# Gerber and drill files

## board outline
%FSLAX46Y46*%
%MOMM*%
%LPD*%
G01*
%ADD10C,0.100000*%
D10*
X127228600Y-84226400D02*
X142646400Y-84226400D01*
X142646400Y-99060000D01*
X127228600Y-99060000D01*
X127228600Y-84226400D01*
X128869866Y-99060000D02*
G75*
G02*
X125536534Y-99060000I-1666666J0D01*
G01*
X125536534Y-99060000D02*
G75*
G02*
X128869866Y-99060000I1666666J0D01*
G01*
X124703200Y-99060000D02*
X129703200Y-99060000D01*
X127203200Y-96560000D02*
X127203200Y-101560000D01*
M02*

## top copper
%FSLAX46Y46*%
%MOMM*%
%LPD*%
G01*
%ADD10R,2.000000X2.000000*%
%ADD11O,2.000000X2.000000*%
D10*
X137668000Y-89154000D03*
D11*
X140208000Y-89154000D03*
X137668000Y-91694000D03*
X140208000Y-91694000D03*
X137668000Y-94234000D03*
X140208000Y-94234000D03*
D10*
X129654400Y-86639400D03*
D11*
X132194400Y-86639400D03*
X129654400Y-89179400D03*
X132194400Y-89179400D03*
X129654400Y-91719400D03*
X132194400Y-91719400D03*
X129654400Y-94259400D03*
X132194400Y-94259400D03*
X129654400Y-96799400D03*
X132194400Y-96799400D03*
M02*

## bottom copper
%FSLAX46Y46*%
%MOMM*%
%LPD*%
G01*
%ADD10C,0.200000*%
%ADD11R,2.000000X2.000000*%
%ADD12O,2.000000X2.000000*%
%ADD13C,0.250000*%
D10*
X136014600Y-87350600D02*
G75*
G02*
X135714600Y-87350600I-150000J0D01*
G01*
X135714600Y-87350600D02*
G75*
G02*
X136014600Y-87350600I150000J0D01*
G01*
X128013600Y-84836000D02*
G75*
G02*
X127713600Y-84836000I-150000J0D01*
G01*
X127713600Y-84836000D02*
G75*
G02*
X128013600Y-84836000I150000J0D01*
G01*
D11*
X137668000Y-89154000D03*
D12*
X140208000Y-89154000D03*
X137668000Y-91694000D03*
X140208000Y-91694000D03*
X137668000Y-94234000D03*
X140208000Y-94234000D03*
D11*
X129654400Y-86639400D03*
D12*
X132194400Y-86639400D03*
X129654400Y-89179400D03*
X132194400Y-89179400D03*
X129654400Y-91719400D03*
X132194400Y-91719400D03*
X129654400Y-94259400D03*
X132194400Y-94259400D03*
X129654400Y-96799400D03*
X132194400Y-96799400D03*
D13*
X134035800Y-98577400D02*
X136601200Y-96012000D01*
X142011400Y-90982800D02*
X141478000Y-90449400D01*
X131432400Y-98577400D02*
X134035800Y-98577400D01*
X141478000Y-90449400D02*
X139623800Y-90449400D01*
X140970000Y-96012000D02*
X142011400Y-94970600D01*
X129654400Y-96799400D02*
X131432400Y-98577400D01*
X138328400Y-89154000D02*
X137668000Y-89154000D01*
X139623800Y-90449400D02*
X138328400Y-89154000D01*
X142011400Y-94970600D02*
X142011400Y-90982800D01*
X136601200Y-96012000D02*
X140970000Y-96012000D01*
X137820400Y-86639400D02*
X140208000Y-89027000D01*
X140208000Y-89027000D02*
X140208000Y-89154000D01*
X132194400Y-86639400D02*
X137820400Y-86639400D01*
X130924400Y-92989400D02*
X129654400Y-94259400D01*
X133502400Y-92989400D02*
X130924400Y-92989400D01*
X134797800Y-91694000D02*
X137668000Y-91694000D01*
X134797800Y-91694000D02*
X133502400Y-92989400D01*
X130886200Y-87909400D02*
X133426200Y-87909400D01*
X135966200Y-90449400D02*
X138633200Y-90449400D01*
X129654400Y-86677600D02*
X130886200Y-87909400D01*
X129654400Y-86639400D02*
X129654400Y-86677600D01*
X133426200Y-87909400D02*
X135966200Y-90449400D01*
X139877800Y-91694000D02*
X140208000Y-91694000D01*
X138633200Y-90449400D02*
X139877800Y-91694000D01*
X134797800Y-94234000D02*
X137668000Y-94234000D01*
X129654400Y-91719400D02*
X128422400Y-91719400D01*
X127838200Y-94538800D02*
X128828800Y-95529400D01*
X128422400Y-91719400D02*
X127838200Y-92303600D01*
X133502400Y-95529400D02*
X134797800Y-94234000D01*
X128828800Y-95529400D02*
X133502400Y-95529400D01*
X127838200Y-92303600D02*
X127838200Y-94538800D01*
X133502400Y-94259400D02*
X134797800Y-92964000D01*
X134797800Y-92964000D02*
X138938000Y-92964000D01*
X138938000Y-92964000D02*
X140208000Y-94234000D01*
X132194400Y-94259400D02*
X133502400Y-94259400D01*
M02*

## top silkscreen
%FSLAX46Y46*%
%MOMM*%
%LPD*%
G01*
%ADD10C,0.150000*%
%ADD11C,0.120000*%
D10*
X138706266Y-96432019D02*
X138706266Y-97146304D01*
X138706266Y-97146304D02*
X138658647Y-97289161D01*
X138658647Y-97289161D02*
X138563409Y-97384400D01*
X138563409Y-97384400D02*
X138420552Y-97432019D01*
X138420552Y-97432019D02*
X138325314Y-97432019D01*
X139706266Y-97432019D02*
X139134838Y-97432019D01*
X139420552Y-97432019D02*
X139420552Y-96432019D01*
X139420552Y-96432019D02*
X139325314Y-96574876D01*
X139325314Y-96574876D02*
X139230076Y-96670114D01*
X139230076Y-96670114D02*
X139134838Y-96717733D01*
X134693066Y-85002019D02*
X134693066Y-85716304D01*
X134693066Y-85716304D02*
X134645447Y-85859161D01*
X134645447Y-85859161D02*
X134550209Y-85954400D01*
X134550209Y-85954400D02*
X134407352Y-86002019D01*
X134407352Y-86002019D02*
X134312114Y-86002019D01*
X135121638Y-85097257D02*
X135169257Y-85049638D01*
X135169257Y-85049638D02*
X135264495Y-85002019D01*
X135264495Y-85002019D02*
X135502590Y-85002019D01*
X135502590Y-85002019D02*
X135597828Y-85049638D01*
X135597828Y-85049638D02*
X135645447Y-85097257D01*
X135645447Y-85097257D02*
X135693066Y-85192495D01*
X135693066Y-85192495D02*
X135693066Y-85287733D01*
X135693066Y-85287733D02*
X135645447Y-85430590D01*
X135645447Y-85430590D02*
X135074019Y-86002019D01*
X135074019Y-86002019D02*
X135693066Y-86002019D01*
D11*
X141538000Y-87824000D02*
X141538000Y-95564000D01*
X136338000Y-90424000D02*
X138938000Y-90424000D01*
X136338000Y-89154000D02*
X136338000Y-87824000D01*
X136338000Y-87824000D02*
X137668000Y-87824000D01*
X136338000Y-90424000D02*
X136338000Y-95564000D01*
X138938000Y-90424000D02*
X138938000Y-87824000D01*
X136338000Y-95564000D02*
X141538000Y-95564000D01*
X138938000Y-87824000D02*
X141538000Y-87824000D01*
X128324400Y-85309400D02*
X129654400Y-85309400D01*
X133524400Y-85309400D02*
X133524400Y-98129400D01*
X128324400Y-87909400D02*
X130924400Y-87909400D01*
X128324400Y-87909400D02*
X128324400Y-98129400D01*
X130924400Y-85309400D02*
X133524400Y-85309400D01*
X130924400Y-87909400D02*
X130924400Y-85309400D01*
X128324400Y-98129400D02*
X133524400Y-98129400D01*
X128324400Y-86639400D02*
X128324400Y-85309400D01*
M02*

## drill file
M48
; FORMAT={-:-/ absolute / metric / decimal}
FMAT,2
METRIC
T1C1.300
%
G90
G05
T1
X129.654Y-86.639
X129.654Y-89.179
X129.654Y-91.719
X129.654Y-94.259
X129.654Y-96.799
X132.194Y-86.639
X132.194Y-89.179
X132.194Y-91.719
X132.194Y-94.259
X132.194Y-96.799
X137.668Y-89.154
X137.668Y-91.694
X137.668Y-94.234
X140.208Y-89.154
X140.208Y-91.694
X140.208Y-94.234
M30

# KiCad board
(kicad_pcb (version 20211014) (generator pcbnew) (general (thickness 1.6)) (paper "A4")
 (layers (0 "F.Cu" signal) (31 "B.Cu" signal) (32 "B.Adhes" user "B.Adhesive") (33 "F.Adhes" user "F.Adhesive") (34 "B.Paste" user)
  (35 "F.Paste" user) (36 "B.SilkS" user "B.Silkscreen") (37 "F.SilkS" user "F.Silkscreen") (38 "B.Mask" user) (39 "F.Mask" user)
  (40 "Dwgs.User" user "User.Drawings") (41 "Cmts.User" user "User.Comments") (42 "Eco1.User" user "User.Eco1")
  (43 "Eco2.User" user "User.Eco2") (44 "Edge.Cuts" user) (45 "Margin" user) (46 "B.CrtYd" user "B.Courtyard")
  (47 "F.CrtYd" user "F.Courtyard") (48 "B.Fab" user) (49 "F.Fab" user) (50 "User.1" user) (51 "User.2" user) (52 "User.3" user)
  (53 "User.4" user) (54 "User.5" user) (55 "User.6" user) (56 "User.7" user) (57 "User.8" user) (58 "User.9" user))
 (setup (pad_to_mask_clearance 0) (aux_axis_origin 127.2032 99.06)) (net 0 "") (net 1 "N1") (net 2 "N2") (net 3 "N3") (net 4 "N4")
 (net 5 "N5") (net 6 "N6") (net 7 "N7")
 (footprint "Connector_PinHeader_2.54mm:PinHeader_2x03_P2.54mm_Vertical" (layer "F.Cu") (at 137.668 89.154)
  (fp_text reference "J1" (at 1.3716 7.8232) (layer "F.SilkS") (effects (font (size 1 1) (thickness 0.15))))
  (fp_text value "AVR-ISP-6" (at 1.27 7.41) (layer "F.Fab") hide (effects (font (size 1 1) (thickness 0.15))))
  (fp_line (start 3.87 -1.33) (end 3.87 6.41) (layer "F.SilkS") (width 0.12))
  (fp_line (start -1.33 1.27) (end 1.27 1.27) (layer "F.SilkS") (width 0.12))
  (fp_line (start -1.33 0) (end -1.33 -1.33) (layer "F.SilkS") (width 0.12))
  (fp_line (start -1.33 -1.33) (end 0 -1.33) (layer "F.SilkS") (width 0.12))
  (fp_line (start -1.33 1.27) (end -1.33 6.41) (layer "F.SilkS") (width 0.12))
  (fp_line (start 1.27 1.27) (end 1.27 -1.33) (layer "F.SilkS") (width 0.12))
  (fp_line (start -1.33 6.41) (end 3.87 6.41) (layer "F.SilkS") (width 0.12))
  (fp_line (start 1.27 -1.33) (end 3.87 -1.33) (layer "F.SilkS") (width 0.12))
  (pad "1" thru_hole rect locked (at 0 0) (size 2 2) (drill 1.3) (layers *.Cu *.Mask) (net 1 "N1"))
  (pad "2" thru_hole oval locked (at 2.54 0) (size 2 2) (drill 1.3) (layers *.Cu *.Mask) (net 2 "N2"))
  (pad "3" thru_hole oval locked (at 0 2.54) (size 2 2) (drill 1.3) (layers *.Cu *.Mask) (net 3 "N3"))
  (pad "4" thru_hole oval locked (at 2.54 2.54) (size 2 2) (drill 1.3) (layers *.Cu *.Mask) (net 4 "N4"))
  (pad "5" thru_hole oval locked (at 0 5.08) (size 2 2) (drill 1.3) (layers *.Cu *.Mask) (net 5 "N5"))
  (pad "6" thru_hole oval locked (at 2.54 5.08) (size 2 2) (drill 1.3) (layers *.Cu *.Mask) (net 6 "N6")))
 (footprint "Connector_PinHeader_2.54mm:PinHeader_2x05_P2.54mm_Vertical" (layer "F.Cu") (at 129.6544 86.6394)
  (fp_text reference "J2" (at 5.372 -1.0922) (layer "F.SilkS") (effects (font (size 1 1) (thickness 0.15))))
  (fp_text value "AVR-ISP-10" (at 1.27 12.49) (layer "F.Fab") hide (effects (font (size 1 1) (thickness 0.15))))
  (fp_line (start -1.33 -1.33) (end 0 -1.33) (layer "F.SilkS") (width 0.12))
  (fp_line (start 3.87 -1.33) (end 3.87 11.49) (layer "F.SilkS") (width 0.12))
  (fp_line (start -1.33 1.27) (end 1.27 1.27) (layer "F.SilkS") (width 0.12))
  (fp_line (start -1.33 1.27) (end -1.33 11.49) (layer "F.SilkS") (width 0.12))
  (fp_line (start 1.27 -1.33) (end 3.87 -1.33) (layer "F.SilkS") (width 0.12))
  (fp_line (start 1.27 1.27) (end 1.27 -1.33) (layer "F.SilkS") (width 0.12))
  (fp_line (start -1.33 11.49) (end 3.87 11.49) (layer "F.SilkS") (width 0.12))
  (fp_line (start -1.33 0) (end -1.33 -1.33) (layer "F.SilkS") (width 0.12))
  (pad "1" thru_hole rect locked (at 0 0) (size 2 2) (drill 1.3) (layers *.Cu *.Mask) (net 4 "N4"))
  (pad "2" thru_hole oval locked (at 2.54 0) (size 2 2) (drill 1.3) (layers *.Cu *.Mask) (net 2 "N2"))
  (pad "3" thru_hole oval locked (at 0 2.54) (size 2 2) (drill 1.3) (layers *.Cu *.Mask) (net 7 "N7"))
  (pad "4" thru_hole oval locked (at 2.54 2.54) (size 2 2) (drill 1.3) (layers *.Cu *.Mask) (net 6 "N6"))
  (pad "5" thru_hole oval locked (at 0 5.08) (size 2 2) (drill 1.3) (layers *.Cu *.Mask) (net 5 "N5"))
  (pad "6" thru_hole oval locked (at 2.54 5.08) (size 2 2) (drill 1.3) (layers *.Cu *.Mask) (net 6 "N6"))
  (pad "7" thru_hole oval locked (at 0 7.62) (size 2 2) (drill 1.3) (layers *.Cu *.Mask) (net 3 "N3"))
  (pad "8" thru_hole oval locked (at 2.54 7.62) (size 2 2) (drill 1.3) (layers *.Cu *.Mask) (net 6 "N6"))
  (pad "9" thru_hole oval locked (at 0 10.16) (size 2 2) (drill 1.3) (layers *.Cu *.Mask) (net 1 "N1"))
  (pad "10" thru_hole oval locked (at 2.54 10.16) (size 2 2) (drill 1.3) (layers *.Cu *.Mask) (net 6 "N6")))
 (gr_circle (center 135.8646 87.3506) (end 136.0146 87.3506) (layer "B.Cu") (width 0.2) (fill none))
 (gr_circle (center 127.8636 84.836) (end 128.0136 84.836) (layer "B.Cu") (width 0.2) (fill none))
 (gr_rect (start 127.2286 84.2264) (end 142.6464 99.06) (layer "Edge.Cuts") (width 0.1) (fill none))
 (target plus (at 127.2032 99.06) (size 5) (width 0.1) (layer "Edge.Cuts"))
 (segment (start 134.0358 98.5774) (end 136.6012 96.012) (width 0.25) (layer "B.Cu") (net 1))
 (segment (start 142.0114 90.9828) (end 141.478 90.4494) (width 0.25) (layer "B.Cu") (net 1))
 (segment (start 131.4324 98.5774) (end 134.0358 98.5774) (width 0.25) (layer "B.Cu") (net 1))
 (segment (start 141.478 90.4494) (end 139.6238 90.4494) (width 0.25) (layer "B.Cu") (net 1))
 (segment (start 140.97 96.012) (end 142.0114 94.9706) (width 0.25) (layer "B.Cu") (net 1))
 (segment (start 129.6544 96.7994) (end 131.4324 98.5774) (width 0.25) (layer "B.Cu") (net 1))
 (segment (start 138.3284 89.154) (end 137.668 89.154) (width 0.25) (layer "B.Cu") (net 1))
 (segment (start 139.6238 90.4494) (end 138.3284 89.154) (width 0.25) (layer "B.Cu") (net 1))
 (segment (start 142.0114 94.9706) (end 142.0114 90.9828) (width 0.25) (layer "B.Cu") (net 1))
 (segment (start 136.6012 96.012) (end 140.97 96.012) (width 0.25) (layer "B.Cu") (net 1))
 (segment (start 137.8204 86.6394) (end 140.208 89.027) (width 0.25) (layer "B.Cu") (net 2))
 (segment (start 140.208 89.027) (end 140.208 89.154) (width 0.25) (layer "B.Cu") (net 2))
 (segment (start 132.1944 86.6394) (end 137.8204 86.6394) (width 0.25) (layer "B.Cu") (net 2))
 (segment (start 130.9244 92.9894) (end 129.6544 94.2594) (width 0.25) (layer "B.Cu") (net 3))
 (segment (start 133.5024 92.9894) (end 130.9244 92.9894) (width 0.25) (layer "B.Cu") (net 3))
 (segment (start 134.7978 91.694) (end 137.668 91.694) (width 0.25) (layer "B.Cu") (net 3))
 (segment (start 134.7978 91.694) (end 133.5024 92.9894) (width 0.25) (layer "B.Cu") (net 3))
 (segment (start 130.8862 87.9094) (end 133.4262 87.9094) (width 0.25) (layer "B.Cu") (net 4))
 (segment (start 135.9662 90.4494) (end 138.6332 90.4494) (width 0.25) (layer "B.Cu") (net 4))
 (segment (start 129.6544 86.6776) (end 130.8862 87.9094) (width 0.25) (layer "B.Cu") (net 4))
 (segment (start 129.6544 86.6394) (end 129.6544 86.6776) (width 0.25) (layer "B.Cu") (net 4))
 (segment (start 133.4262 87.9094) (end 135.9662 90.4494) (width 0.25) (layer "B.Cu") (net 4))
 (segment (start 139.8778 91.694) (end 140.208 91.694) (width 0.25) (layer "B.Cu") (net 4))
 (segment (start 138.6332 90.4494) (end 139.8778 91.694) (width 0.25) (layer "B.Cu") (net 4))
 (segment (start 134.7978 94.234) (end 137.668 94.234) (width 0.25) (layer "B.Cu") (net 5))
 (segment (start 129.6544 91.7194) (end 128.4224 91.7194) (width 0.25) (layer "B.Cu") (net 5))
 (segment (start 127.8382 94.5388) (end 128.8288 95.5294) (width 0.25) (layer "B.Cu") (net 5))
 (segment (start 128.4224 91.7194) (end 127.8382 92.3036) (width 0.25) (layer "B.Cu") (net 5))
 (segment (start 133.5024 95.5294) (end 134.7978 94.234) (width 0.25) (layer "B.Cu") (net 5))
 (segment (start 128.8288 95.5294) (end 133.5024 95.5294) (width 0.25) (layer "B.Cu") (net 5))
 (segment (start 127.8382 92.3036) (end 127.8382 94.5388) (width 0.25) (layer "B.Cu") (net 5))
 (segment (start 133.5024 94.2594) (end 134.7978 92.964) (width 0.25) (layer "B.Cu") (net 6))
 (segment (start 134.7978 92.964) (end 138.938 92.964) (width 0.25) (layer "B.Cu") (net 6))
 (segment (start 138.938 92.964) (end 140.208 94.234) (width 0.25) (layer "B.Cu") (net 6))
 (segment (start 132.1944 94.2594) (end 133.5024 94.2594) (width 0.25) (layer "B.Cu") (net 6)))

